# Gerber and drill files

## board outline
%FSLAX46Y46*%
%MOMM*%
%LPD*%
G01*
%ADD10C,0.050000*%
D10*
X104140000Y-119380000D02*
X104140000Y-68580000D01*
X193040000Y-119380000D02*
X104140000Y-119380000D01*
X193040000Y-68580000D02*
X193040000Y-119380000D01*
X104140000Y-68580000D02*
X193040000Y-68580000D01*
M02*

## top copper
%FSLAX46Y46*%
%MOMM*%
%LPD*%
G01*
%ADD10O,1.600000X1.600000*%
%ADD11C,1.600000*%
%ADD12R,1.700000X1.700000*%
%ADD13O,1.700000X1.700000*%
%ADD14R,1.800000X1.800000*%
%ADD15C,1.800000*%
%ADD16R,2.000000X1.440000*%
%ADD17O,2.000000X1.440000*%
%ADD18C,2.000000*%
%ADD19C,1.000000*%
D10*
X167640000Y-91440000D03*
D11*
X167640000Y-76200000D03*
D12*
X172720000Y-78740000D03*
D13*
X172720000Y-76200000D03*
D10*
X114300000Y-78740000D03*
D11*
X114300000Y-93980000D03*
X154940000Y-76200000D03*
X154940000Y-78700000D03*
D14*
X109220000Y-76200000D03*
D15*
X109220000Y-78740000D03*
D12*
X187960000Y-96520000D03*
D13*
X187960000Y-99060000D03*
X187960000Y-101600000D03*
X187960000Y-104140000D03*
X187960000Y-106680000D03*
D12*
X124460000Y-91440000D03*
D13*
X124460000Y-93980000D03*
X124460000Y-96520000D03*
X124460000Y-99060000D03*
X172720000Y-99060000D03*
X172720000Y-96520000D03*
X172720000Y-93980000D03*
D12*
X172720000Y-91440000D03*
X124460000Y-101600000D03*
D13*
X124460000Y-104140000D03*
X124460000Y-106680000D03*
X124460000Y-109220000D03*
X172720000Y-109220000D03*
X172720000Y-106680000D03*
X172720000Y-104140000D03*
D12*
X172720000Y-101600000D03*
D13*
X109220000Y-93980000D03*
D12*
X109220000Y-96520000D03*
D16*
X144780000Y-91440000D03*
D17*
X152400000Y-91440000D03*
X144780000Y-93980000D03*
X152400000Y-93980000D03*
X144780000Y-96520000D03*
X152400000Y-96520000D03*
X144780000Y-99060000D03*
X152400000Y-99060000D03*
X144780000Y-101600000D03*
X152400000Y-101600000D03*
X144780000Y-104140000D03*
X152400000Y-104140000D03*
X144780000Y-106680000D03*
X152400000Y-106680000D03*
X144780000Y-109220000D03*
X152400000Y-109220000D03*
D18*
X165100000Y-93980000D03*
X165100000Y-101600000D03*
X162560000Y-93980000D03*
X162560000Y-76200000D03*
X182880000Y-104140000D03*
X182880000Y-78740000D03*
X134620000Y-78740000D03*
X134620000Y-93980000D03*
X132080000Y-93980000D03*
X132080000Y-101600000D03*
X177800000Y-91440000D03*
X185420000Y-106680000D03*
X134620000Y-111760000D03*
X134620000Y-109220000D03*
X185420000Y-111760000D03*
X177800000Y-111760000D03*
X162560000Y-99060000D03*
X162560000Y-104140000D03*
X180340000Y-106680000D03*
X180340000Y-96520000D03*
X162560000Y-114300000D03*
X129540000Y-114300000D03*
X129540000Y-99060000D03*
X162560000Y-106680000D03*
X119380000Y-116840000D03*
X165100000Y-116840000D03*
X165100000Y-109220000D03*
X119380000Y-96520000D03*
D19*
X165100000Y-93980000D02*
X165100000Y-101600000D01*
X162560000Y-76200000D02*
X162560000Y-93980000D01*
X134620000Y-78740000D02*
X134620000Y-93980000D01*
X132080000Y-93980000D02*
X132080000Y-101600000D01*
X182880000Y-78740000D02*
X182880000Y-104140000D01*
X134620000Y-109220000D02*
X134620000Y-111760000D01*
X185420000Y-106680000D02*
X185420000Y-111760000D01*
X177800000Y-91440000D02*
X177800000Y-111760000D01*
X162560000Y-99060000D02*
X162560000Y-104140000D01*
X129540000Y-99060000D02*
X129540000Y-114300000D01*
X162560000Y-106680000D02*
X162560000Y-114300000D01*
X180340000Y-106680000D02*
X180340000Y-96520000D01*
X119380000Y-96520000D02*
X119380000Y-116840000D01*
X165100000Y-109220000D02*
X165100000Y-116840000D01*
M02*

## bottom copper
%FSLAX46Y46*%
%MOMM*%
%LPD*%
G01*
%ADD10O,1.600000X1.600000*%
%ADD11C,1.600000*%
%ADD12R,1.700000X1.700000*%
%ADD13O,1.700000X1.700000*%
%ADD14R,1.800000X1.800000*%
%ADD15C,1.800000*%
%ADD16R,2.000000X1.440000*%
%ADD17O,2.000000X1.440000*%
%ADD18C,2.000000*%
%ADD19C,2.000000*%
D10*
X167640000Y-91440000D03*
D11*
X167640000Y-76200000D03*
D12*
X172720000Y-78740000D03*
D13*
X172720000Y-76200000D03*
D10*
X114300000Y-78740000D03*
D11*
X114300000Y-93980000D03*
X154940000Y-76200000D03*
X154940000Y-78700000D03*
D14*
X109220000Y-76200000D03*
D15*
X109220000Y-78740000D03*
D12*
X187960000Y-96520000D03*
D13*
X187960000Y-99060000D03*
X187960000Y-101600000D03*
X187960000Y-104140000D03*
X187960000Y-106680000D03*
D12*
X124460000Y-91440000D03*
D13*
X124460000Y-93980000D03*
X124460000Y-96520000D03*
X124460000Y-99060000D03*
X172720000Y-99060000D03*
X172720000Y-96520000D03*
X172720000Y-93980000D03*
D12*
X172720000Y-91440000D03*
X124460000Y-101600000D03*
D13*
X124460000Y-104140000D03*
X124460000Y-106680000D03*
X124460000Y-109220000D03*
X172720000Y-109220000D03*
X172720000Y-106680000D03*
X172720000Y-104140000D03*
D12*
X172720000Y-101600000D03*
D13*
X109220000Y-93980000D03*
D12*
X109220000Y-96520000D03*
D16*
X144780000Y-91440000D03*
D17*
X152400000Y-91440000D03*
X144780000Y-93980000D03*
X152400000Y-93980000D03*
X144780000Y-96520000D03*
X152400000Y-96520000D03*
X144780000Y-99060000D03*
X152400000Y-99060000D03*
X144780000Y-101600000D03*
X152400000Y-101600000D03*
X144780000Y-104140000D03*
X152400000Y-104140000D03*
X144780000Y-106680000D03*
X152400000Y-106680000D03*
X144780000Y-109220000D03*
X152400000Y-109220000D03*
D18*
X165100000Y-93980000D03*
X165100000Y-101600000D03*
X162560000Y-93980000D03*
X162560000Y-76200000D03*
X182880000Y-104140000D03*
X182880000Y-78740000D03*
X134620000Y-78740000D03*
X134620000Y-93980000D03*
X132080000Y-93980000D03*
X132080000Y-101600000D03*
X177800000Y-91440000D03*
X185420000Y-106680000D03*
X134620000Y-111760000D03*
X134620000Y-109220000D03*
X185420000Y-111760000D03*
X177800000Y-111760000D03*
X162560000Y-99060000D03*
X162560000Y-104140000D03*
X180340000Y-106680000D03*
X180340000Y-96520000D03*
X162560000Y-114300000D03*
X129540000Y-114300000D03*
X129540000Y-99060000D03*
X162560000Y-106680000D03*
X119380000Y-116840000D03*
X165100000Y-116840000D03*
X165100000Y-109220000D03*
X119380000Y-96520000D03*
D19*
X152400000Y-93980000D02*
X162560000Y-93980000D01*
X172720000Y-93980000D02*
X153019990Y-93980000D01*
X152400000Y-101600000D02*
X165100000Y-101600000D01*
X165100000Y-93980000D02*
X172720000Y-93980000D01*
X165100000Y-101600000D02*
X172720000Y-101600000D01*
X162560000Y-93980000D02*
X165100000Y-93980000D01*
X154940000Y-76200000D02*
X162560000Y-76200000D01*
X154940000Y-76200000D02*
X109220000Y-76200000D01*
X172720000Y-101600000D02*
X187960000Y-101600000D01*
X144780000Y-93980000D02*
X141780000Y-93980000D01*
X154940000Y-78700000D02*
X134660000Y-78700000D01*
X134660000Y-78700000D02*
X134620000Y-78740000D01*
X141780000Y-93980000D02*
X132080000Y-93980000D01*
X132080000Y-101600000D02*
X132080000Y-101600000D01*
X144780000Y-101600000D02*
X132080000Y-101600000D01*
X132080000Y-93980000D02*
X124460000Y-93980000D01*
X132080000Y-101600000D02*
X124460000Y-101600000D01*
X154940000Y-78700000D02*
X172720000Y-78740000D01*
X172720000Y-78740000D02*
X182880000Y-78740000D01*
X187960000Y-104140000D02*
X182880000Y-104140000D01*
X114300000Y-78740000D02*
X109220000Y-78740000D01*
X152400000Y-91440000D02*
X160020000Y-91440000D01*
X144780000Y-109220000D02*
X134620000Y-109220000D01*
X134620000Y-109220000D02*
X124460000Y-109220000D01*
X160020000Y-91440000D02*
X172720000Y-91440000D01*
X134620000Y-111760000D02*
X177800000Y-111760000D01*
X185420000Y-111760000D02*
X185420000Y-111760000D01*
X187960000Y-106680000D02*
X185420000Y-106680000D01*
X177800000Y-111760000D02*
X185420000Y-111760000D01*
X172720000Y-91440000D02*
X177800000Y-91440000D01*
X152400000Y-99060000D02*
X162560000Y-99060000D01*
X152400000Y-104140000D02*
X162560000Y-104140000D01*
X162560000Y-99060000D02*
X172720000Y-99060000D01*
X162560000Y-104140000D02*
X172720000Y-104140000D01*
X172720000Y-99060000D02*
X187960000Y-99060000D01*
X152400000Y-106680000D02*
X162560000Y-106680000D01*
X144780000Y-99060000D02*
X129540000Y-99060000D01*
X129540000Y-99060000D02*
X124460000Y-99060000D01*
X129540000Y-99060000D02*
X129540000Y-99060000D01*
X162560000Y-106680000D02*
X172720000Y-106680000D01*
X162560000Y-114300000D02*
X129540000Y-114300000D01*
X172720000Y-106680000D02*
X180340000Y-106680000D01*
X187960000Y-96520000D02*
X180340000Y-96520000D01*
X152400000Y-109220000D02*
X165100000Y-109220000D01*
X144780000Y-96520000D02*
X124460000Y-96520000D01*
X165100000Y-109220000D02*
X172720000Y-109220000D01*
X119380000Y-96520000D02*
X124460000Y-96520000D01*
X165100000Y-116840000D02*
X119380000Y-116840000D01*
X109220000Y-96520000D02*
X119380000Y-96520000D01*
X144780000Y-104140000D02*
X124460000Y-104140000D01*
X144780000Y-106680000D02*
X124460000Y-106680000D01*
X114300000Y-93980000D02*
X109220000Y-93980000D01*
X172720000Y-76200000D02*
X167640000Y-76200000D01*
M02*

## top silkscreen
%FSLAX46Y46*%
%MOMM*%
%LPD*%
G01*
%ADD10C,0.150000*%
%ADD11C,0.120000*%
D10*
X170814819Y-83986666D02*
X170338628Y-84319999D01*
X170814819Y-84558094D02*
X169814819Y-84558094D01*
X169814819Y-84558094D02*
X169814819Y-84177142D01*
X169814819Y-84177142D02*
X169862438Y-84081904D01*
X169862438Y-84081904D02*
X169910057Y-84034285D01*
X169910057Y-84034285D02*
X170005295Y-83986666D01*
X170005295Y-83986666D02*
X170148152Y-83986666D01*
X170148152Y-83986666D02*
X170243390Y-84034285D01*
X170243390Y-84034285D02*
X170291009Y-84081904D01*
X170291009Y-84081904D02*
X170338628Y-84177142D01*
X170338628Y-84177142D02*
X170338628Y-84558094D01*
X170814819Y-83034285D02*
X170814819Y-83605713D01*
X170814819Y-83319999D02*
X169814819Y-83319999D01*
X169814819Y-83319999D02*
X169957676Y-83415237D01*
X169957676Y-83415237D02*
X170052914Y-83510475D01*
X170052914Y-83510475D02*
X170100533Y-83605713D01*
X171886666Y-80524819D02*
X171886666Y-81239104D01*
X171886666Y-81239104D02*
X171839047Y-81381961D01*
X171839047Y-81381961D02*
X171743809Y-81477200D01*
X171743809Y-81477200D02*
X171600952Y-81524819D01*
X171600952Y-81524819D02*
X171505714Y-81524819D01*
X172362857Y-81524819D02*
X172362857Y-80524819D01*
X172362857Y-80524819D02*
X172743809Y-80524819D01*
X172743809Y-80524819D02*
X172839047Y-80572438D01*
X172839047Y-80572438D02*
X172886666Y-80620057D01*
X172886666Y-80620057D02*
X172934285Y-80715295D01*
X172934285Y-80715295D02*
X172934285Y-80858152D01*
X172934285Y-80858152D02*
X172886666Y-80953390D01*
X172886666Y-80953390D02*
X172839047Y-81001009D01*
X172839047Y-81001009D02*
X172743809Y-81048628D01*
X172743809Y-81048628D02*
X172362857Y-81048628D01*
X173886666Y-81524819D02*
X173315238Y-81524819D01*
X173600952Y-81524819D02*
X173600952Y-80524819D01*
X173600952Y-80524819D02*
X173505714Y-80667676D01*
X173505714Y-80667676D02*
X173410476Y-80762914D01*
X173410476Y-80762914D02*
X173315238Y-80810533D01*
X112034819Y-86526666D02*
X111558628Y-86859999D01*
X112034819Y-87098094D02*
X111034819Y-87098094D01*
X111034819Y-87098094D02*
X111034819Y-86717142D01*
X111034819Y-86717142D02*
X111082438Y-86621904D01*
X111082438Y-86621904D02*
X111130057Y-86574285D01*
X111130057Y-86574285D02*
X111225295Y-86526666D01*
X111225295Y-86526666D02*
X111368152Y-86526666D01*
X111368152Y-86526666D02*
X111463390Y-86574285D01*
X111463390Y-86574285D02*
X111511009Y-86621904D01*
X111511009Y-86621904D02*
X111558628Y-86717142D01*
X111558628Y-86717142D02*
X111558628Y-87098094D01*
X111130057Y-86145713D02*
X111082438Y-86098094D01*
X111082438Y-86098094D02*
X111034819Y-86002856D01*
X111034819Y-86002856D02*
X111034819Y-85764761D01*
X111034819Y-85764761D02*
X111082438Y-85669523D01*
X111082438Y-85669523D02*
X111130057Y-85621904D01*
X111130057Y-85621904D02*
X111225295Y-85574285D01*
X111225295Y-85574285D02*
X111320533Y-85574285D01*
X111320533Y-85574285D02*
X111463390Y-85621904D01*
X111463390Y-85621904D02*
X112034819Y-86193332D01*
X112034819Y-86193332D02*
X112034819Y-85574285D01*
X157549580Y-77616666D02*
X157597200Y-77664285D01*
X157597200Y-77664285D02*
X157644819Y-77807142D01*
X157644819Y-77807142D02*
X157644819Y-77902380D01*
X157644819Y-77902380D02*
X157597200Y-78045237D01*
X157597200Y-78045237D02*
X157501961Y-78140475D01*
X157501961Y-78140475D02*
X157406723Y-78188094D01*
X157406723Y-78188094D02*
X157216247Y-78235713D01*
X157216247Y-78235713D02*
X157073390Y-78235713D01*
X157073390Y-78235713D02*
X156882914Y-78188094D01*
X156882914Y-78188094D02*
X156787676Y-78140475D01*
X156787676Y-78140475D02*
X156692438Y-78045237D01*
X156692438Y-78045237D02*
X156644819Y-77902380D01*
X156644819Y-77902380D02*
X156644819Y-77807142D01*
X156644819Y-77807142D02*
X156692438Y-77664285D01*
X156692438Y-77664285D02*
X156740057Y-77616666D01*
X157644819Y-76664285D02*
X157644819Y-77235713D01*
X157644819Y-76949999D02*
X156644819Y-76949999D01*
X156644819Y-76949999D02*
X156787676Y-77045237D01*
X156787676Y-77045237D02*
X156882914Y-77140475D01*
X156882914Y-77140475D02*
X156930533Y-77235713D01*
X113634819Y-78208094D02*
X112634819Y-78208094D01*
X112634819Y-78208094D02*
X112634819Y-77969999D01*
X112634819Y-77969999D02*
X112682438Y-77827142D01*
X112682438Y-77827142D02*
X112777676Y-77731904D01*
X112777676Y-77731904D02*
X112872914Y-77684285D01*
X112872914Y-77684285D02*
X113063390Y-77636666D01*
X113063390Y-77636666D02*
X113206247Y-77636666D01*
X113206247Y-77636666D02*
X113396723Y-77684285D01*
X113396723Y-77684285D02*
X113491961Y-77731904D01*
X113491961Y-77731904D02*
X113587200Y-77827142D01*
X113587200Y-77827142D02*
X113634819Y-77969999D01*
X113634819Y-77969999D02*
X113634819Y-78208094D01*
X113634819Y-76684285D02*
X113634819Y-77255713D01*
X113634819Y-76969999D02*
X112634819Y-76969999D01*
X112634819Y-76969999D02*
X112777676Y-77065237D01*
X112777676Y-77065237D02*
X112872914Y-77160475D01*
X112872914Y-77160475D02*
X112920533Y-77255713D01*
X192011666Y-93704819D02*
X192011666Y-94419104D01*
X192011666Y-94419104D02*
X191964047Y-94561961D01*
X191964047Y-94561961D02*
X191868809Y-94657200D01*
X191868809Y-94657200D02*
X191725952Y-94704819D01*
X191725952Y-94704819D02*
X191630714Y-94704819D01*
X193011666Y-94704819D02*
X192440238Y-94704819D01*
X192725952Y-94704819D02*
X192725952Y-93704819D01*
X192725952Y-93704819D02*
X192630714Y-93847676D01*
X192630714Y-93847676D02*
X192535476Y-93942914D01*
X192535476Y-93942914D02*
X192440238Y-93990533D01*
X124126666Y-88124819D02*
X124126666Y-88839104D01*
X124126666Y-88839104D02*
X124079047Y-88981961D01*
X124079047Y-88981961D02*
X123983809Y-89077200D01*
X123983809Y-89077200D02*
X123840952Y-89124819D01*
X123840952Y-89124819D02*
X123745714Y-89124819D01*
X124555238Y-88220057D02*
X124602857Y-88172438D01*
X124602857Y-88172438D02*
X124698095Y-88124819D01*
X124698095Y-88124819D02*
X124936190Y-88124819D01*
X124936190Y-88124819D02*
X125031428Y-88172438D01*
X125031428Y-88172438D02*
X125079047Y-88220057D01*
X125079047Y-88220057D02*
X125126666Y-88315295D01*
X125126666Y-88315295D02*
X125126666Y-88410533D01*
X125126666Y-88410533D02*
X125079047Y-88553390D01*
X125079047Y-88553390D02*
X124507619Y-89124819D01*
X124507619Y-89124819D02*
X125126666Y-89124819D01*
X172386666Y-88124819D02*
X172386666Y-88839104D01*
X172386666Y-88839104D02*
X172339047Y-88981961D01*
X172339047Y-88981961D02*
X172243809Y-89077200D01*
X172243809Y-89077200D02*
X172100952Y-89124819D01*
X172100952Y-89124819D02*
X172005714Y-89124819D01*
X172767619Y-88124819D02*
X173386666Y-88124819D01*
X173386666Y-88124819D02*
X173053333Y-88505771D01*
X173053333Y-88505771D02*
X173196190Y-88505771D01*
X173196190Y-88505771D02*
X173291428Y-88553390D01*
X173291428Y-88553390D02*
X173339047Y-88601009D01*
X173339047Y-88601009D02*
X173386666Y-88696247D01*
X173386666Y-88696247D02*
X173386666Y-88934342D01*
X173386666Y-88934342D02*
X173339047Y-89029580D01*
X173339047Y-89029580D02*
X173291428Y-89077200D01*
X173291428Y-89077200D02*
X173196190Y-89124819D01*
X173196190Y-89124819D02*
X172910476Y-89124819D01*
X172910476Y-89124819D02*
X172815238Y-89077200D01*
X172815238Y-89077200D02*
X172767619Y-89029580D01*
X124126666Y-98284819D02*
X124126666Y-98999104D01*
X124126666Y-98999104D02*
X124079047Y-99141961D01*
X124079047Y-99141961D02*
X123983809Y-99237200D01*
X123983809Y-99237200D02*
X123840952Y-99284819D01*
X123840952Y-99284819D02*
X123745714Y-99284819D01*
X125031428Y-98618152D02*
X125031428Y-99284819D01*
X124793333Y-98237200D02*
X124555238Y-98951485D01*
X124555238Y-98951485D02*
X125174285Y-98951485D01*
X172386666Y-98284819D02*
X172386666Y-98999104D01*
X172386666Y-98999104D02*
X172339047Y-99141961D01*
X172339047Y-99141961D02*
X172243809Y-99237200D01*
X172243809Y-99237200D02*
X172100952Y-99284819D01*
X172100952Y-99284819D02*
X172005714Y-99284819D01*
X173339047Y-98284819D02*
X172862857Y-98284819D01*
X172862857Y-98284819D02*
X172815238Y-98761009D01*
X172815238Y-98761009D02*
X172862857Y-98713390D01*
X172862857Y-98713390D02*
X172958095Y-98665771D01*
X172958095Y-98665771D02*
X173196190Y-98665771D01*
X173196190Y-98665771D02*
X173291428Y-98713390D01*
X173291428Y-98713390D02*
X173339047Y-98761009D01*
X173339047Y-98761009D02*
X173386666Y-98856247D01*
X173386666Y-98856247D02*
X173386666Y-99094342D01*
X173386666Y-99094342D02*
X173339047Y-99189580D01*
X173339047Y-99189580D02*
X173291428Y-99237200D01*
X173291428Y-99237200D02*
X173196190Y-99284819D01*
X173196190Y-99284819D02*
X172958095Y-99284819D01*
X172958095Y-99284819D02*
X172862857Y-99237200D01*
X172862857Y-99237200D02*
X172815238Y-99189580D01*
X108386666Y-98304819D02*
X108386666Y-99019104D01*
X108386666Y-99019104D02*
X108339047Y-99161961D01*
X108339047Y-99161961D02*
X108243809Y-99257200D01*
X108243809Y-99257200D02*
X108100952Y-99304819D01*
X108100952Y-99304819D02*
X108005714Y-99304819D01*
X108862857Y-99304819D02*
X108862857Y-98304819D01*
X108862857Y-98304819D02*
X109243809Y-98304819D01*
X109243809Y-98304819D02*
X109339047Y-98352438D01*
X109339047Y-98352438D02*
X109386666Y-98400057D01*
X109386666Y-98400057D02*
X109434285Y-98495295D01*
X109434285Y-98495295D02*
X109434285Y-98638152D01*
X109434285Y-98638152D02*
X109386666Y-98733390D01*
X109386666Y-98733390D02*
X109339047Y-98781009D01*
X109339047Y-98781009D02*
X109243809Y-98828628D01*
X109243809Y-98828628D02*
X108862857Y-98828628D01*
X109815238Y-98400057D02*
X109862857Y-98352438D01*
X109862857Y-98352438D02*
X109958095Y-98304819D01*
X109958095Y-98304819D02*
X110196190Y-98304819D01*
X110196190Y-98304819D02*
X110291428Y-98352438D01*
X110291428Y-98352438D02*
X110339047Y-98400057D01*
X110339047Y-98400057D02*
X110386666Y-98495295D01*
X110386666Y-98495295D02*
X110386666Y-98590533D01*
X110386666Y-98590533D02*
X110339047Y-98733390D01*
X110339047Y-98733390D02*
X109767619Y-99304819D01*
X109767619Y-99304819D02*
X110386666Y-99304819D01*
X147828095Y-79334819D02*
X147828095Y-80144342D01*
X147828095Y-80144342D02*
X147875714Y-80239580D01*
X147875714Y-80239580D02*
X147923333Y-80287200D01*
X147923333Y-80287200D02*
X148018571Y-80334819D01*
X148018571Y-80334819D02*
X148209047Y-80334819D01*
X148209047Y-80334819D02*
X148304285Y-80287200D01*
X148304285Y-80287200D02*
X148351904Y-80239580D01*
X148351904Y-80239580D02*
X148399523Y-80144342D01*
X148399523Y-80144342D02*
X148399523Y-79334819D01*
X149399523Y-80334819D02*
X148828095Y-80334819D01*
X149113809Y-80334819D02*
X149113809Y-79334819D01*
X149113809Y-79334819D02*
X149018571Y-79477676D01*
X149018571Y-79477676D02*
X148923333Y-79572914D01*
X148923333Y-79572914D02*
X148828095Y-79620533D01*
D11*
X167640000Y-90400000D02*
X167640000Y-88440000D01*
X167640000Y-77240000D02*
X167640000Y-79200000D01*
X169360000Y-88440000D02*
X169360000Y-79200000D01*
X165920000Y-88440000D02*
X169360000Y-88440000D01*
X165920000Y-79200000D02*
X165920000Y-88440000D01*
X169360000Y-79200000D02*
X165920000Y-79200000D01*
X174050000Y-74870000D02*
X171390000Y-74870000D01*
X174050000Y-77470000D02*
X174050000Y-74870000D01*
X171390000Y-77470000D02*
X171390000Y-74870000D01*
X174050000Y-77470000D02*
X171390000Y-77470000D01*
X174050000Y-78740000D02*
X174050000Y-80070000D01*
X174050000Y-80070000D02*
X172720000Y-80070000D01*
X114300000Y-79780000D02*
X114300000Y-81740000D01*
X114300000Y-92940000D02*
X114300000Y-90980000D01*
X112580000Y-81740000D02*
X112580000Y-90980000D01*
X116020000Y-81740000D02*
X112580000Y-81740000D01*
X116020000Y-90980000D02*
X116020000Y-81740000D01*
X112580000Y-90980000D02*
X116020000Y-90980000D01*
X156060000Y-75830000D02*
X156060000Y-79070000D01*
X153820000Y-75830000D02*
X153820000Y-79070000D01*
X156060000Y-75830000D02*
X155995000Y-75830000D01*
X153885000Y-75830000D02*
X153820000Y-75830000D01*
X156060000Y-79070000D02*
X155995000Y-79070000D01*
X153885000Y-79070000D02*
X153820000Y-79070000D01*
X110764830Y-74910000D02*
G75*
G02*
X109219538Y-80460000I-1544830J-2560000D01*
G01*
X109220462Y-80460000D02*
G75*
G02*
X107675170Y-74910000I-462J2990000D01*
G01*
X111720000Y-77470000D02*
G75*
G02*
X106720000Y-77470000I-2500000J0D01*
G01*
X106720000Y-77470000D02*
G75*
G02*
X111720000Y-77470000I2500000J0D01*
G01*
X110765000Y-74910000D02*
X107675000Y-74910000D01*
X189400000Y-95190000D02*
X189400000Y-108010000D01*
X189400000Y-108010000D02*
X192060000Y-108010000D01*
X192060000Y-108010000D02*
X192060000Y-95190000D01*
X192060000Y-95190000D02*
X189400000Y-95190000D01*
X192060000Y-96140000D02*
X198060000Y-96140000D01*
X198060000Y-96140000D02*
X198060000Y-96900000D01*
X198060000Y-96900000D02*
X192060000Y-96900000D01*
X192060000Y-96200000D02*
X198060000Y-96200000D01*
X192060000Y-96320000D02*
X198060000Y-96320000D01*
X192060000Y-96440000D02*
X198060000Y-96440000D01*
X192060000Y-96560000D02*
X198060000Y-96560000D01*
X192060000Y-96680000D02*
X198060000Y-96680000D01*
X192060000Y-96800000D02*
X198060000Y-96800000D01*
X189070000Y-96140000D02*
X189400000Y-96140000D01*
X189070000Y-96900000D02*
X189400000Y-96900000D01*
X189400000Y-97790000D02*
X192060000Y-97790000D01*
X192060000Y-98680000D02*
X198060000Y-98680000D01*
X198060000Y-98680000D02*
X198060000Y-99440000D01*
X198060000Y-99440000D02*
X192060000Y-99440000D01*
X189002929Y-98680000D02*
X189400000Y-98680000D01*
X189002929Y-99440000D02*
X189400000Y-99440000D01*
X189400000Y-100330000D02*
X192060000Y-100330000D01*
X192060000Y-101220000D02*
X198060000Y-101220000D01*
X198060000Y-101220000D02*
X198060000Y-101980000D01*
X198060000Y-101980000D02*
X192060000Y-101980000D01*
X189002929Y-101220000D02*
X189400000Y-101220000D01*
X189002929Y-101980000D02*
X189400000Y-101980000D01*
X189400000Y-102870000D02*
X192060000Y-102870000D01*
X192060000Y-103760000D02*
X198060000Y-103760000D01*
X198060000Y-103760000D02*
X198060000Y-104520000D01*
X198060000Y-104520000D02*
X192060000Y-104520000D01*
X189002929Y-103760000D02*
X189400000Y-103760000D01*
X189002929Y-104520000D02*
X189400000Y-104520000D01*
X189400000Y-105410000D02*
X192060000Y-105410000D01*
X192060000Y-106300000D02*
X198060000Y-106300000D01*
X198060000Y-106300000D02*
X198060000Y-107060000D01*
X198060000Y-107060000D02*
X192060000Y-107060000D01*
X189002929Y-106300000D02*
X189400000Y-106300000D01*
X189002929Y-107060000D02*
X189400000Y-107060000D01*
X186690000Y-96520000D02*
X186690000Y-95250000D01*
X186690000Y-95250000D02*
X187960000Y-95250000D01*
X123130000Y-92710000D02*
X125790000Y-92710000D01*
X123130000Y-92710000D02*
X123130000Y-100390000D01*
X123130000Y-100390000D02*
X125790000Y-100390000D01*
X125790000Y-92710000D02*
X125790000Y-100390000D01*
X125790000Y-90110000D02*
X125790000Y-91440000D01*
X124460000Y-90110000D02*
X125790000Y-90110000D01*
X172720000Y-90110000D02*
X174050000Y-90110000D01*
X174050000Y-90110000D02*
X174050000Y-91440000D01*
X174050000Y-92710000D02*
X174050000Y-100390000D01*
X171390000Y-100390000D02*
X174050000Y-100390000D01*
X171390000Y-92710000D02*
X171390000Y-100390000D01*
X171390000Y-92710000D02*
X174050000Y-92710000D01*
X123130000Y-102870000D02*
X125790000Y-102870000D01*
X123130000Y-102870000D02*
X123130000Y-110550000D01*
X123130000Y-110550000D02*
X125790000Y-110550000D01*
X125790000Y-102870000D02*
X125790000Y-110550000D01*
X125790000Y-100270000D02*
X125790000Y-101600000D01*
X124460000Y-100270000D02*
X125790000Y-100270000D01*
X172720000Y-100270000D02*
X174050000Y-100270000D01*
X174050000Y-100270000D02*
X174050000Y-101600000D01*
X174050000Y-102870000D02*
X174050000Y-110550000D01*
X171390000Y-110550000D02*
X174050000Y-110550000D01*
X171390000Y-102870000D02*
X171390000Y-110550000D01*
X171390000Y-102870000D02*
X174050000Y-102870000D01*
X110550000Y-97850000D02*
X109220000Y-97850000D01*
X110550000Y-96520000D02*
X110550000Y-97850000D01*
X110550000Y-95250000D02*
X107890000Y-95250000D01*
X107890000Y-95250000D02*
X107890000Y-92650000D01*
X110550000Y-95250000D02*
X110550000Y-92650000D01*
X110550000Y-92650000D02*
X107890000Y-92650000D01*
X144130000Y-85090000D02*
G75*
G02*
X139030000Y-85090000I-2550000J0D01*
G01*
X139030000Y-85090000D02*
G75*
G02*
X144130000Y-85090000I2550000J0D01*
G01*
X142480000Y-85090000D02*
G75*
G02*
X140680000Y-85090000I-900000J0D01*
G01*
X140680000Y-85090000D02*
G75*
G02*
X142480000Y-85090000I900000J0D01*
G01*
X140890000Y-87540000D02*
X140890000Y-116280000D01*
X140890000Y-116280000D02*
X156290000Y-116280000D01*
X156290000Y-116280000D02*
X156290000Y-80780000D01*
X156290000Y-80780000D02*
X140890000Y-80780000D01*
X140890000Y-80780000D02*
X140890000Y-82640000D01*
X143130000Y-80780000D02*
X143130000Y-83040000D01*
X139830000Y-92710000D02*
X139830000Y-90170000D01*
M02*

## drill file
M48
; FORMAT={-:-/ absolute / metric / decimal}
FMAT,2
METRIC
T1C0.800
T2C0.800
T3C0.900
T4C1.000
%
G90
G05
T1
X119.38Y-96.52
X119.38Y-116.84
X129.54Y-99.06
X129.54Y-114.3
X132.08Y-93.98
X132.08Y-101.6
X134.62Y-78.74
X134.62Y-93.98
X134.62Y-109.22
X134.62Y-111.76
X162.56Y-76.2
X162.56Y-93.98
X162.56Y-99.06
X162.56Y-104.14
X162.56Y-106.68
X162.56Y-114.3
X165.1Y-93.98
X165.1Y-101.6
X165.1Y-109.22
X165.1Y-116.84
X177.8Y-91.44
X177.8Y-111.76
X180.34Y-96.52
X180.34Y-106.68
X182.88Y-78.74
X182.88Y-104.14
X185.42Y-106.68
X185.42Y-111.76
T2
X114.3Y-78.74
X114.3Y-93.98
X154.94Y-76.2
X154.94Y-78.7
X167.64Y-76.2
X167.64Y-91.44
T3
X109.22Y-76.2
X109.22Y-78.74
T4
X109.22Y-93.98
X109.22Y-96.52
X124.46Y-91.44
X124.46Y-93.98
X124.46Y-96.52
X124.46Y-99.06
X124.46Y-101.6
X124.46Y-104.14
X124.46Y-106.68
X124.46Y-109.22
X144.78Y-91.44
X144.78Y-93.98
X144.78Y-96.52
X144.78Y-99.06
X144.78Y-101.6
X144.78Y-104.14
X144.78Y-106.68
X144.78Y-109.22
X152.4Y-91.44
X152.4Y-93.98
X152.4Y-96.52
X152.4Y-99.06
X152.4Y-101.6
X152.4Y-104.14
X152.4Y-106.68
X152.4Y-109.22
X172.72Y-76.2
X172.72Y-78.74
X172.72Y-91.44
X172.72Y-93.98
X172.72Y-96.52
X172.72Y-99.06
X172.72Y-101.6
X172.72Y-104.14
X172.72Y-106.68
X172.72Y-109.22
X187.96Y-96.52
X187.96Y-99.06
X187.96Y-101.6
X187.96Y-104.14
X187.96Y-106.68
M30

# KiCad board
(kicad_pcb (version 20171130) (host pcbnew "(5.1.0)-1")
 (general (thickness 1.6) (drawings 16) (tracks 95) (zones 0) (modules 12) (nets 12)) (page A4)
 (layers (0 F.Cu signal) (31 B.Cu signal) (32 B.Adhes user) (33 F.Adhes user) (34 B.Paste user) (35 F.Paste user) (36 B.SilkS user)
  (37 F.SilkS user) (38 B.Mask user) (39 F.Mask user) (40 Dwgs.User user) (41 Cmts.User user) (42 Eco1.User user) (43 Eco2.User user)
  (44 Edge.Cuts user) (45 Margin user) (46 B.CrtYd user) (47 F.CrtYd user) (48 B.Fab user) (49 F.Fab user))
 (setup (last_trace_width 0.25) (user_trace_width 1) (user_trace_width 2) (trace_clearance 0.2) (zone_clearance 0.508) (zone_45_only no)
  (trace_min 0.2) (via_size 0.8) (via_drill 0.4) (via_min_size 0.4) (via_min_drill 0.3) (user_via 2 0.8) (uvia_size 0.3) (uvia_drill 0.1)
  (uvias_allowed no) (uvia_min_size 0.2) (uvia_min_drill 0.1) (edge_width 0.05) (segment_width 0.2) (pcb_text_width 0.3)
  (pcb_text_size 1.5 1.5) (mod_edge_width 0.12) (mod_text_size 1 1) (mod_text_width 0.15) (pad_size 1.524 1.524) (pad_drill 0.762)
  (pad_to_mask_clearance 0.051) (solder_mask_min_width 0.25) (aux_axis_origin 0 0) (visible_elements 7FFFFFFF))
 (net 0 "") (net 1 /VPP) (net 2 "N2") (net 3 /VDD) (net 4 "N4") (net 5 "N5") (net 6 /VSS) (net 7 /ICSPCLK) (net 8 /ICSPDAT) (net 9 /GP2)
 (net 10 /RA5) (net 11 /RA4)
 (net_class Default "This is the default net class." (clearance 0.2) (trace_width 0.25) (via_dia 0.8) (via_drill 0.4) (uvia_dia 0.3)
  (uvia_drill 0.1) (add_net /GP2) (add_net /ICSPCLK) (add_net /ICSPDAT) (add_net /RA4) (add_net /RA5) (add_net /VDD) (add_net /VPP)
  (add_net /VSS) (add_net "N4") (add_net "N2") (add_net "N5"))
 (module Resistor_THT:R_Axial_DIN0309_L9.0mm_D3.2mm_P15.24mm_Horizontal (layer F.Cu) (at 167.64 76.2 270)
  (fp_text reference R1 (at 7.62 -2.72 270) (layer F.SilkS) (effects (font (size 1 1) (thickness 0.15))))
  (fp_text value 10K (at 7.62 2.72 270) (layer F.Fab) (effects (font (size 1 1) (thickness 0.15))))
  (fp_line (start 14.2 0) (end 12.24 0) (layer F.SilkS) (width 0.12))
  (fp_line (start 1.04 0) (end 3 0) (layer F.SilkS) (width 0.12))
  (fp_line (start 12.24 -1.72) (end 3 -1.72) (layer F.SilkS) (width 0.12))
  (fp_line (start 12.24 1.72) (end 12.24 -1.72) (layer F.SilkS) (width 0.12))
  (fp_line (start 3 1.72) (end 12.24 1.72) (layer F.SilkS) (width 0.12))
  (fp_line (start 3 -1.72) (end 3 1.72) (layer F.SilkS) (width 0.12))
  (pad 2 thru_hole oval (at 15.24 0 270) (size 1.6 1.6) (drill 0.8) (layers *.Cu *.Mask) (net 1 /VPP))
  (pad 1 thru_hole circle (at 0 0 270) (size 1.6 1.6) (drill 0.8) (layers *.Cu *.Mask) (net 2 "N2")))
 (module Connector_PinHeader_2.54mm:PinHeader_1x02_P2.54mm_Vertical (layer F.Cu) (at 172.72 78.74 180)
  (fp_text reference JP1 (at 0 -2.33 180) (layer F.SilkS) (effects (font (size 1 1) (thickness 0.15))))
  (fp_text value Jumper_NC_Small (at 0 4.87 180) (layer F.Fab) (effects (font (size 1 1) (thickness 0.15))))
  (fp_line (start -1.33 3.87) (end 1.33 3.87) (layer F.SilkS) (width 0.12))
  (fp_line (start -1.33 1.27) (end -1.33 3.87) (layer F.SilkS) (width 0.12))
  (fp_line (start 1.33 1.27) (end 1.33 3.87) (layer F.SilkS) (width 0.12))
  (fp_line (start -1.33 1.27) (end 1.33 1.27) (layer F.SilkS) (width 0.12))
  (fp_line (start -1.33 0) (end -1.33 -1.33) (layer F.SilkS) (width 0.12))
  (fp_line (start -1.33 -1.33) (end 0 -1.33) (layer F.SilkS) (width 0.12))
  (pad 1 thru_hole rect (at 0 0 180) (size 1.7 1.7) (drill 1) (layers *.Cu *.Mask) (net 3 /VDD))
  (pad 2 thru_hole oval (at 0 2.54 180) (size 1.7 1.7) (drill 1) (layers *.Cu *.Mask) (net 2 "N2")))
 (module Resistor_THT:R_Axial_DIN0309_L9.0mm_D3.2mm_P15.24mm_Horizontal (layer F.Cu) (at 114.3 93.98 90)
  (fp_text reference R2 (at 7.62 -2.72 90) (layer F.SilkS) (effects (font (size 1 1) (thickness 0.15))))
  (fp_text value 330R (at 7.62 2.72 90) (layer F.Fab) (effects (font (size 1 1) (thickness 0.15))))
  (fp_line (start 14.2 0) (end 12.24 0) (layer F.SilkS) (width 0.12))
  (fp_line (start 1.04 0) (end 3 0) (layer F.SilkS) (width 0.12))
  (fp_line (start 12.24 -1.72) (end 3 -1.72) (layer F.SilkS) (width 0.12))
  (fp_line (start 12.24 1.72) (end 12.24 -1.72) (layer F.SilkS) (width 0.12))
  (fp_line (start 3 1.72) (end 12.24 1.72) (layer F.SilkS) (width 0.12))
  (fp_line (start 3 -1.72) (end 3 1.72) (layer F.SilkS) (width 0.12))
  (pad 2 thru_hole oval (at 15.24 0 90) (size 1.6 1.6) (drill 0.8) (layers *.Cu *.Mask) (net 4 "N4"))
  (pad 1 thru_hole circle (at 0 0 90) (size 1.6 1.6) (drill 0.8) (layers *.Cu *.Mask) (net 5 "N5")))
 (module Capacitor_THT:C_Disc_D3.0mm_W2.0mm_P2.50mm (layer F.Cu) (at 154.94 76.2 270)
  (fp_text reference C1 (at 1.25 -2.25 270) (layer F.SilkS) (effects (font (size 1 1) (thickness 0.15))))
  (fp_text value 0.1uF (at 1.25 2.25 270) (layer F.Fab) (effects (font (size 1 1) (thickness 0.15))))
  (fp_line (start -0.37 -1.12) (end 2.87 -1.12) (layer F.SilkS) (width 0.12))
  (fp_line (start -0.37 1.12) (end 2.87 1.12) (layer F.SilkS) (width 0.12))
  (fp_line (start -0.37 -1.12) (end -0.37 -1.055) (layer F.SilkS) (width 0.12))
  (fp_line (start -0.37 1.055) (end -0.37 1.12) (layer F.SilkS) (width 0.12))
  (fp_line (start 2.87 -1.12) (end 2.87 -1.055) (layer F.SilkS) (width 0.12))
  (fp_line (start 2.87 1.055) (end 2.87 1.12) (layer F.SilkS) (width 0.12))
  (pad 1 thru_hole circle (at 0 0 270) (size 1.6 1.6) (drill 0.8) (layers *.Cu *.Mask) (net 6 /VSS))
  (pad 2 thru_hole circle (at 2.5 0 270) (size 1.6 1.6) (drill 0.8) (layers *.Cu *.Mask) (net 3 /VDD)))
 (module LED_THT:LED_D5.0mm (layer F.Cu) (at 109.22 76.2 270)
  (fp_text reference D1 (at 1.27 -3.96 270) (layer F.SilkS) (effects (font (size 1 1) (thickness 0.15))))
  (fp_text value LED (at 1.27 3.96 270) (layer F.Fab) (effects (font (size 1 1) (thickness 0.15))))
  (fp_arc (start 1.27 0) (end -1.29 -1.54483) (angle 148.9) (layer F.SilkS) (width 0.12))
  (fp_arc (start 1.27 0) (end -1.29 1.54483) (angle -148.9) (layer F.SilkS) (width 0.12))
  (fp_circle (center 1.27 0) (end 3.77 0) (layer F.SilkS) (width 0.12))
  (fp_line (start -1.29 -1.545) (end -1.29 1.545) (layer F.SilkS) (width 0.12))
  (pad 1 thru_hole rect (at 0 0 270) (size 1.8 1.8) (drill 0.9) (layers *.Cu *.Mask) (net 6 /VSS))
  (pad 2 thru_hole circle (at 2.54 0 270) (size 1.8 1.8) (drill 0.9) (layers *.Cu *.Mask) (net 4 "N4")))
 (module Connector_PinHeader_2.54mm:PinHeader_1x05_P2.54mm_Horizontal (layer F.Cu) (at 187.96 96.52)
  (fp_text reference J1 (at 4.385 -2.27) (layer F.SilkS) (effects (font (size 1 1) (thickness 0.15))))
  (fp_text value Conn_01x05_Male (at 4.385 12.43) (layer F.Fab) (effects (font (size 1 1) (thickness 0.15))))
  (fp_line (start 1.44 -1.33) (end 1.44 11.49) (layer F.SilkS) (width 0.12))
  (fp_line (start 1.44 11.49) (end 4.1 11.49) (layer F.SilkS) (width 0.12))
  (fp_line (start 4.1 11.49) (end 4.1 -1.33) (layer F.SilkS) (width 0.12))
  (fp_line (start 4.1 -1.33) (end 1.44 -1.33) (layer F.SilkS) (width 0.12))
  (fp_line (start 4.1 -0.38) (end 10.1 -0.38) (layer F.SilkS) (width 0.12))
  (fp_line (start 10.1 -0.38) (end 10.1 0.38) (layer F.SilkS) (width 0.12))
  (fp_line (start 10.1 0.38) (end 4.1 0.38) (layer F.SilkS) (width 0.12))
  (fp_line (start 4.1 -0.32) (end 10.1 -0.32) (layer F.SilkS) (width 0.12))
  (fp_line (start 4.1 -0.2) (end 10.1 -0.2) (layer F.SilkS) (width 0.12))
  (fp_line (start 4.1 -0.08) (end 10.1 -0.08) (layer F.SilkS) (width 0.12))
  (fp_line (start 4.1 0.04) (end 10.1 0.04) (layer F.SilkS) (width 0.12))
  (fp_line (start 4.1 0.16) (end 10.1 0.16) (layer F.SilkS) (width 0.12))
  (fp_line (start 4.1 0.28) (end 10.1 0.28) (layer F.SilkS) (width 0.12))
  (fp_line (start 1.11 -0.38) (end 1.44 -0.38) (layer F.SilkS) (width 0.12))
  (fp_line (start 1.11 0.38) (end 1.44 0.38) (layer F.SilkS) (width 0.12))
  (fp_line (start 1.44 1.27) (end 4.1 1.27) (layer F.SilkS) (width 0.12))
  (fp_line (start 4.1 2.16) (end 10.1 2.16) (layer F.SilkS) (width 0.12))
  (fp_line (start 10.1 2.16) (end 10.1 2.92) (layer F.SilkS) (width 0.12))
  (fp_line (start 10.1 2.92) (end 4.1 2.92) (layer F.SilkS) (width 0.12))
  (fp_line (start 1.042929 2.16) (end 1.44 2.16) (layer F.SilkS) (width 0.12))
  (fp_line (start 1.042929 2.92) (end 1.44 2.92) (layer F.SilkS) (width 0.12))
  (fp_line (start 1.44 3.81) (end 4.1 3.81) (layer F.SilkS) (width 0.12))
  (fp_line (start 4.1 4.7) (end 10.1 4.7) (layer F.SilkS) (width 0.12))
  (fp_line (start 10.1 4.7) (end 10.1 5.46) (layer F.SilkS) (width 0.12))
  (fp_line (start 10.1 5.46) (end 4.1 5.46) (layer F.SilkS) (width 0.12))
  (fp_line (start 1.042929 4.7) (end 1.44 4.7) (layer F.SilkS) (width 0.12))
  (fp_line (start 1.042929 5.46) (end 1.44 5.46) (layer F.SilkS) (width 0.12))
  (fp_line (start 1.44 6.35) (end 4.1 6.35) (layer F.SilkS) (width 0.12))
  (fp_line (start 4.1 7.24) (end 10.1 7.24) (layer F.SilkS) (width 0.12))
  (fp_line (start 10.1 7.24) (end 10.1 8) (layer F.SilkS) (width 0.12))
  (fp_line (start 10.1 8) (end 4.1 8) (layer F.SilkS) (width 0.12))
  (fp_line (start 1.042929 7.24) (end 1.44 7.24) (layer F.SilkS) (width 0.12))
  (fp_line (start 1.042929 8) (end 1.44 8) (layer F.SilkS) (width 0.12))
  (fp_line (start 1.44 8.89) (end 4.1 8.89) (layer F.SilkS) (width 0.12))
  (fp_line (start 4.1 9.78) (end 10.1 9.78) (layer F.SilkS) (width 0.12))
  (fp_line (start 10.1 9.78) (end 10.1 10.54) (layer F.SilkS) (width 0.12))
  (fp_line (start 10.1 10.54) (end 4.1 10.54) (layer F.SilkS) (width 0.12))
  (fp_line (start 1.042929 9.78) (end 1.44 9.78) (layer F.SilkS) (width 0.12))
  (fp_line (start 1.042929 10.54) (end 1.44 10.54) (layer F.SilkS) (width 0.12))
  (fp_line (start -1.27 0) (end -1.27 -1.27) (layer F.SilkS) (width 0.12))
  (fp_line (start -1.27 -1.27) (end 0 -1.27) (layer F.SilkS) (width 0.12))
  (pad 1 thru_hole rect (at 0 0) (size 1.7 1.7) (drill 1) (layers *.Cu *.Mask) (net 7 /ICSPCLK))
  (pad 2 thru_hole oval (at 0 2.54) (size 1.7 1.7) (drill 1) (layers *.Cu *.Mask) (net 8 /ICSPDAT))
  (pad 3 thru_hole oval (at 0 5.08) (size 1.7 1.7) (drill 1) (layers *.Cu *.Mask) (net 6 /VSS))
  (pad 4 thru_hole oval (at 0 7.62) (size 1.7 1.7) (drill 1) (layers *.Cu *.Mask) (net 3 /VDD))
  (pad 5 thru_hole oval (at 0 10.16) (size 1.7 1.7) (drill 1) (layers *.Cu *.Mask) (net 1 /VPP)))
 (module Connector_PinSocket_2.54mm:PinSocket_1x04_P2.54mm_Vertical (layer F.Cu) (at 124.46 91.44)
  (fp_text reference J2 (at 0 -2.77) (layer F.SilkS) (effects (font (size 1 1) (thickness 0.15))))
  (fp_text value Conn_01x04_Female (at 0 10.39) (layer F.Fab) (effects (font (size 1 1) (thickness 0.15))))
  (fp_line (start -1.33 1.27) (end 1.33 1.27) (layer F.SilkS) (width 0.12))
  (fp_line (start -1.33 1.27) (end -1.33 8.95) (layer F.SilkS) (width 0.12))
  (fp_line (start -1.33 8.95) (end 1.33 8.95) (layer F.SilkS) (width 0.12))
  (fp_line (start 1.33 1.27) (end 1.33 8.95) (layer F.SilkS) (width 0.12))
  (fp_line (start 1.33 -1.33) (end 1.33 0) (layer F.SilkS) (width 0.12))
  (fp_line (start 0 -1.33) (end 1.33 -1.33) (layer F.SilkS) (width 0.12))
  (pad 1 thru_hole rect (at 0 0) (size 1.7 1.7) (drill 1) (layers *.Cu *.Mask))
  (pad 2 thru_hole oval (at 0 2.54) (size 1.7 1.7) (drill 1) (layers *.Cu *.Mask) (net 3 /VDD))
  (pad 3 thru_hole oval (at 0 5.08) (size 1.7 1.7) (drill 1) (layers *.Cu *.Mask) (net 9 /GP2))
  (pad 4 thru_hole oval (at 0 7.62) (size 1.7 1.7) (drill 1) (layers *.Cu *.Mask) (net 7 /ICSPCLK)))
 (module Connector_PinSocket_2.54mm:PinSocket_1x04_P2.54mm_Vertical (layer F.Cu) (at 172.72 91.44)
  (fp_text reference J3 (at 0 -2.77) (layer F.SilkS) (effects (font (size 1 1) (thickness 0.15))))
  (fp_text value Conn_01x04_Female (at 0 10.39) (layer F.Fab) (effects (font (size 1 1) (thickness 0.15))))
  (fp_line (start 0 -1.33) (end 1.33 -1.33) (layer F.SilkS) (width 0.12))
  (fp_line (start 1.33 -1.33) (end 1.33 0) (layer F.SilkS) (width 0.12))
  (fp_line (start 1.33 1.27) (end 1.33 8.95) (layer F.SilkS) (width 0.12))
  (fp_line (start -1.33 8.95) (end 1.33 8.95) (layer F.SilkS) (width 0.12))
  (fp_line (start -1.33 1.27) (end -1.33 8.95) (layer F.SilkS) (width 0.12))
  (fp_line (start -1.33 1.27) (end 1.33 1.27) (layer F.SilkS) (width 0.12))
  (pad 4 thru_hole oval (at 0 7.62) (size 1.7 1.7) (drill 1) (layers *.Cu *.Mask) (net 8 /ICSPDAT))
  (pad 3 thru_hole oval (at 0 5.08) (size 1.7 1.7) (drill 1) (layers *.Cu *.Mask))
  (pad 2 thru_hole oval (at 0 2.54) (size 1.7 1.7) (drill 1) (layers *.Cu *.Mask) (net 6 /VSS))
  (pad 1 thru_hole rect (at 0 0) (size 1.7 1.7) (drill 1) (layers *.Cu *.Mask) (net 1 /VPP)))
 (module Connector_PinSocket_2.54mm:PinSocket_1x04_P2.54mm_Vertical (layer F.Cu) (at 124.46 101.6)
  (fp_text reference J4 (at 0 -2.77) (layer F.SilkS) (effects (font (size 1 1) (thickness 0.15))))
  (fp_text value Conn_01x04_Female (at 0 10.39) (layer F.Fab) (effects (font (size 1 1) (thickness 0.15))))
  (fp_line (start -1.33 1.27) (end 1.33 1.27) (layer F.SilkS) (width 0.12))
  (fp_line (start -1.33 1.27) (end -1.33 8.95) (layer F.SilkS) (width 0.12))
  (fp_line (start -1.33 8.95) (end 1.33 8.95) (layer F.SilkS) (width 0.12))
  (fp_line (start 1.33 1.27) (end 1.33 8.95) (layer F.SilkS) (width 0.12))
  (fp_line (start 1.33 -1.33) (end 1.33 0) (layer F.SilkS) (width 0.12))
  (fp_line (start 0 -1.33) (end 1.33 -1.33) (layer F.SilkS) (width 0.12))
  (pad 1 thru_hole rect (at 0 0) (size 1.7 1.7) (drill 1) (layers *.Cu *.Mask) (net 3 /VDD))
  (pad 2 thru_hole oval (at 0 2.54) (size 1.7 1.7) (drill 1) (layers *.Cu *.Mask) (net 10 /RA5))
  (pad 3 thru_hole oval (at 0 5.08) (size 1.7 1.7) (drill 1) (layers *.Cu *.Mask) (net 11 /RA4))
  (pad 4 thru_hole oval (at 0 7.62) (size 1.7 1.7) (drill 1) (layers *.Cu *.Mask) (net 1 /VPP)))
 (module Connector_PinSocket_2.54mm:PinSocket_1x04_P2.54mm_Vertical (layer F.Cu) (at 172.72 101.6)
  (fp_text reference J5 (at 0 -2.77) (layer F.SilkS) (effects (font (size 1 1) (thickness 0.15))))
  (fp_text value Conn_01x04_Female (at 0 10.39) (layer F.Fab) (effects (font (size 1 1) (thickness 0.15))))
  (fp_line (start 0 -1.33) (end 1.33 -1.33) (layer F.SilkS) (width 0.12))
  (fp_line (start 1.33 -1.33) (end 1.33 0) (layer F.SilkS) (width 0.12))
  (fp_line (start 1.33 1.27) (end 1.33 8.95) (layer F.SilkS) (width 0.12))
  (fp_line (start -1.33 8.95) (end 1.33 8.95) (layer F.SilkS) (width 0.12))
  (fp_line (start -1.33 1.27) (end -1.33 8.95) (layer F.SilkS) (width 0.12))
  (fp_line (start -1.33 1.27) (end 1.33 1.27) (layer F.SilkS) (width 0.12))
  (pad 4 thru_hole oval (at 0 7.62) (size 1.7 1.7) (drill 1) (layers *.Cu *.Mask) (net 9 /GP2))
  (pad 3 thru_hole oval (at 0 5.08) (size 1.7 1.7) (drill 1) (layers *.Cu *.Mask) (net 7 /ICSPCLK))
  (pad 2 thru_hole oval (at 0 2.54) (size 1.7 1.7) (drill 1) (layers *.Cu *.Mask) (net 8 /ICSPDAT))
  (pad 1 thru_hole rect (at 0 0) (size 1.7 1.7) (drill 1) (layers *.Cu *.Mask) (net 6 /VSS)))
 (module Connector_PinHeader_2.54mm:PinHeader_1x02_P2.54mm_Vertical (layer F.Cu) (at 109.22 96.52 180)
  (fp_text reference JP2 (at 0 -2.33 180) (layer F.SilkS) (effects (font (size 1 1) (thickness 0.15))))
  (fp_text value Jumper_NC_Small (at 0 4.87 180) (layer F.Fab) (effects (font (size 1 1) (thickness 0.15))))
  (fp_line (start -1.33 -1.33) (end 0 -1.33) (layer F.SilkS) (width 0.12))
  (fp_line (start -1.33 0) (end -1.33 -1.33) (layer F.SilkS) (width 0.12))
  (fp_line (start -1.33 1.27) (end 1.33 1.27) (layer F.SilkS) (width 0.12))
  (fp_line (start 1.33 1.27) (end 1.33 3.87) (layer F.SilkS) (width 0.12))
  (fp_line (start -1.33 1.27) (end -1.33 3.87) (layer F.SilkS) (width 0.12))
  (fp_line (start -1.33 3.87) (end 1.33 3.87) (layer F.SilkS) (width 0.12))
  (pad 2 thru_hole oval (at 0 2.54 180) (size 1.7 1.7) (drill 1) (layers *.Cu *.Mask) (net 5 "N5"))
  (pad 1 thru_hole rect (at 0 0 180) (size 1.7 1.7) (drill 1) (layers *.Cu *.Mask) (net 9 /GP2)))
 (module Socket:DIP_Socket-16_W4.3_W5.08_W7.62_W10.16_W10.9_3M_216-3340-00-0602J (layer F.Cu) (at 144.78 91.44)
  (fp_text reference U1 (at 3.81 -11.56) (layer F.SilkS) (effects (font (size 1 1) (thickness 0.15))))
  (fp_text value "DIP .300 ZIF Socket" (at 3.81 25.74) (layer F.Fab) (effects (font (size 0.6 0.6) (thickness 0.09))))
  (fp_circle (center -3.2 -6.35) (end -0.65 -6.35) (layer F.SilkS) (width 0.12))
  (fp_circle (center -3.2 -6.35) (end -2.3 -6.35) (layer F.SilkS) (width 0.12))
  (fp_line (start -3.89 -3.9) (end -3.89 24.84) (layer F.SilkS) (width 0.12))
  (fp_line (start -3.89 24.84) (end 11.51 24.84) (layer F.SilkS) (width 0.12))
  (fp_line (start 11.51 24.84) (end 11.51 -10.66) (layer F.SilkS) (width 0.12))
  (fp_line (start 11.51 -10.66) (end -3.89 -10.66) (layer F.SilkS) (width 0.12))
  (fp_line (start -3.89 -10.66) (end -3.89 -8.8) (layer F.SilkS) (width 0.12))
  (fp_line (start -1.65 -10.66) (end -1.65 -8.4) (layer F.SilkS) (width 0.12))
  (fp_line (start -4.95 1.27) (end -4.95 -1.27) (layer F.SilkS) (width 0.12))
  (pad 1 thru_hole rect (at 0 0) (size 2 1.44) (drill 1) (layers *.Cu *.Mask))
  (pad 16 thru_hole oval (at 7.62 0) (size 2 1.44) (drill 1) (layers *.Cu *.Mask) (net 1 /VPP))
  (pad 2 thru_hole oval (at 0 2.54) (size 2 1.44) (drill 1) (layers *.Cu *.Mask) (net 3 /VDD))
  (pad 15 thru_hole oval (at 7.62 2.54) (size 2 1.44) (drill 1) (layers *.Cu *.Mask) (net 6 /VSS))
  (pad 3 thru_hole oval (at 0 5.08) (size 2 1.44) (drill 1) (layers *.Cu *.Mask) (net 9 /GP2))
  (pad 14 thru_hole oval (at 7.62 5.08) (size 2 1.44) (drill 1) (layers *.Cu *.Mask))
  (pad 4 thru_hole oval (at 0 7.62) (size 2 1.44) (drill 1) (layers *.Cu *.Mask) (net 7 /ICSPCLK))
  (pad 13 thru_hole oval (at 7.62 7.62) (size 2 1.44) (drill 1) (layers *.Cu *.Mask) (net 8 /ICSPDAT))
  (pad 5 thru_hole oval (at 0 10.16) (size 2 1.44) (drill 1) (layers *.Cu *.Mask) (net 3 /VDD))
  (pad 12 thru_hole oval (at 7.62 10.16) (size 2 1.44) (drill 1) (layers *.Cu *.Mask) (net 6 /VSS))
  (pad 6 thru_hole oval (at 0 12.7) (size 2 1.44) (drill 1) (layers *.Cu *.Mask) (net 10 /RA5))
  (pad 11 thru_hole oval (at 7.62 12.7) (size 2 1.44) (drill 1) (layers *.Cu *.Mask) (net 8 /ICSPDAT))
  (pad 7 thru_hole oval (at 0 15.24) (size 2 1.44) (drill 1) (layers *.Cu *.Mask) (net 11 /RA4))
  (pad 10 thru_hole oval (at 7.62 15.24) (size 2 1.44) (drill 1) (layers *.Cu *.Mask) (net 7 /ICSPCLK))
  (pad 8 thru_hole oval (at 0 17.78) (size 2 1.44) (drill 1) (layers *.Cu *.Mask) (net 1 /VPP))
  (pad 9 thru_hole oval (at 7.62 17.78) (size 2 1.44) (drill 1) (layers *.Cu *.Mask) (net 9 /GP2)))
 (gr_line (start 104.14 119.38) (end 104.14 68.58) (layer Edge.Cuts) (width 0.05))
 (gr_line (start 193.04 119.38) (end 104.14 119.38) (layer Edge.Cuts) (width 0.05))
 (gr_line (start 193.04 68.58) (end 193.04 119.38) (layer Edge.Cuts) (width 0.05))
 (gr_line (start 104.14 68.58) (end 193.04 68.58) (layer Edge.Cuts) (width 0.05))
 (segment (start 152.4 93.98) (end 162.56 93.98) (width 2) (layer B.Cu) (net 6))
 (segment (start 172.72 93.98) (end 153.01999 93.98) (width 2) (layer B.Cu) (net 6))
 (segment (start 152.4 101.6) (end 165.1 101.6) (width 2) (layer B.Cu) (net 6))
 (segment (start 165.1 93.98) (end 172.72 93.98) (width 2) (layer B.Cu) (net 6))
 (via (at 165.1 93.98) (size 2) (drill 0.8) (layers F.Cu B.Cu) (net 6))
 (segment (start 165.1 101.6) (end 172.72 101.6) (width 2) (layer B.Cu) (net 6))
 (via (at 165.1 101.6) (size 2) (drill 0.8) (layers F.Cu B.Cu) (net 6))
 (segment (start 165.1 93.98) (end 165.1 101.6) (width 1) (layer F.Cu) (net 6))
 (segment (start 162.56 93.98) (end 165.1 93.98) (width 2) (layer B.Cu) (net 6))
 (via (at 162.56 93.98) (size 2) (drill 0.8) (layers F.Cu B.Cu) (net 6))
 (segment (start 154.94 76.2) (end 162.56 76.2) (width 2) (layer B.Cu) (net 6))
 (via (at 162.56 76.2) (size 2) (drill 0.8) (layers F.Cu B.Cu) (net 6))
 (segment (start 162.56 76.2) (end 162.56 93.98) (width 1) (layer F.Cu) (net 6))
 (segment (start 154.94 76.2) (end 109.22 76.2) (width 2) (layer B.Cu) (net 6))
 (segment (start 172.72 101.6) (end 187.96 101.6) (width 2) (layer B.Cu) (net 6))
 (via (at 182.88 104.14) (size 2) (drill 0.8) (layers F.Cu B.Cu) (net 3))
 (via (at 182.88 78.74) (size 2) (drill 0.8) (layers F.Cu B.Cu) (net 3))
 (segment (start 144.78 93.98) (end 141.78 93.98) (width 2) (layer B.Cu) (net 3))
 (via (at 134.62 78.74) (size 2) (drill 0.8) (layers F.Cu B.Cu) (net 3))
 (segment (start 154.94 78.7) (end 134.66 78.7) (width 2) (layer B.Cu) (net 3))
 (segment (start 134.66 78.7) (end 134.62 78.74) (width 2) (layer B.Cu) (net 3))
 (segment (start 134.62 78.74) (end 134.62 93.98) (width 1) (layer F.Cu) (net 3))
 (segment (start 141.78 93.98) (end 132.08 93.98) (width 2) (layer B.Cu) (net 3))
 (via (at 134.62 93.98) (size 2) (drill 0.8) (layers F.Cu B.Cu) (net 3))
 (segment (start 132.08 101.6) (end 132.08 101.6) (width 2) (layer B.Cu) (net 3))
 (segment (start 144.78 101.6) (end 132.08 101.6) (width 2) (layer B.Cu) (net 3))
 (segment (start 132.08 93.98) (end 124.46 93.98) (width 2) (layer B.Cu) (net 3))
 (via (at 132.08 93.98) (size 2) (drill 0.8) (layers F.Cu B.Cu) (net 3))
 (segment (start 132.08 101.6) (end 124.46 101.6) (width 2) (layer B.Cu) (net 3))
 (via (at 132.08 101.6) (size 2) (drill 0.8) (layers F.Cu B.Cu) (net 3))
 (segment (start 132.08 93.98) (end 132.08 101.6) (width 1) (layer F.Cu) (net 3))
 (segment (start 154.94 78.7) (end 172.72 78.74) (width 2) (layer B.Cu) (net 3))
 (segment (start 172.72 78.74) (end 182.88 78.74) (width 2) (layer B.Cu) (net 3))
 (segment (start 182.88 78.74) (end 182.88 104.14) (width 1) (layer F.Cu) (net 3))
 (segment (start 187.96 104.14) (end 182.88 104.14) (width 2) (layer B.Cu) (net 3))
 (segment (start 114.3 78.74) (end 109.22 78.74) (width 2) (layer B.Cu) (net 4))
 (via (at 177.8 91.44) (size 2) (drill 0.8) (layers F.Cu B.Cu) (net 1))
 (via (at 185.42 106.68) (size 2) (drill 0.8) (layers F.Cu B.Cu) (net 1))
 (via (at 134.62 111.76) (size 2) (drill 0.8) (layers F.Cu B.Cu) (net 1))
 (segment (start 152.4 91.44) (end 160.02 91.44) (width 2) (layer B.Cu) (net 1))
 (segment (start 144.78 109.22) (end 134.62 109.22) (width 2) (layer B.Cu) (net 1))
 (segment (start 134.62 109.22) (end 124.46 109.22) (width 2) (layer B.Cu) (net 1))
 (via (at 134.62 109.22) (size 2) (drill 0.8) (layers F.Cu B.Cu) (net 1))
 (segment (start 134.62 109.22) (end 134.62 111.76) (width 1) (layer F.Cu) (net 1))
 (segment (start 160.02 91.44) (end 172.72 91.44) (width 2) (layer B.Cu) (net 1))
 (segment (start 134.62 111.76) (end 177.8 111.76) (width 2) (layer B.Cu) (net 1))
 (segment (start 185.42 111.76) (end 185.42 111.76) (width 2) (layer B.Cu) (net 1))
 (via (at 185.42 111.76) (size 2) (drill 0.8) (layers F.Cu B.Cu) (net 1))
 (segment (start 187.96 106.68) (end 185.42 106.68) (width 2) (layer B.Cu) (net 1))
 (segment (start 185.42 106.68) (end 185.42 111.76) (width 1) (layer F.Cu) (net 1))
 (segment (start 177.8 111.76) (end 185.42 111.76) (width 2) (layer B.Cu) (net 1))
 (via (at 177.8 111.76) (size 2) (drill 0.8) (layers F.Cu B.Cu) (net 1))
 (segment (start 172.72 91.44) (end 177.8 91.44) (width 2) (layer B.Cu) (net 1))
 (segment (start 177.8 91.44) (end 177.8 111.76) (width 1) (layer F.Cu) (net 1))
 (segment (start 152.4 99.06) (end 162.56 99.06) (width 2) (layer B.Cu) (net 8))
 (segment (start 152.4 104.14) (end 162.56 104.14) (width 2) (layer B.Cu) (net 8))
 (segment (start 162.56 99.06) (end 172.72 99.06) (width 2) (layer B.Cu) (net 8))
 (via (at 162.56 99.06) (size 2) (drill 0.8) (layers F.Cu B.Cu) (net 8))
 (segment (start 162.56 104.14) (end 172.72 104.14) (width 2) (layer B.Cu) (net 8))
 (via (at 162.56 104.14) (size 2) (drill 0.8) (layers F.Cu B.Cu) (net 8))
 (segment (start 162.56 99.06) (end 162.56 104.14) (width 1) (layer F.Cu) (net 8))
 (segment (start 172.72 99.06) (end 187.96 99.06) (width 2) (layer B.Cu) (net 8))
 (via (at 180.34 106.68) (size 2) (drill 0.8) (layers F.Cu B.Cu) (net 7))
 (via (at 180.34 96.52) (size 2) (drill 0.8) (layers F.Cu B.Cu) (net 7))
 (via (at 162.56 114.3) (size 2) (drill 0.8) (layers F.Cu B.Cu) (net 7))
 (via (at 129.54 114.3) (size 2) (drill 0.8) (layers F.Cu B.Cu) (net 7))
 (segment (start 152.4 106.68) (end 162.56 106.68) (width 2) (layer B.Cu) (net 7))
 (segment (start 144.78 99.06) (end 129.54 99.06) (width 2) (layer B.Cu) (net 7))
 (segment (start 129.54 99.06) (end 124.46 99.06) (width 2) (layer B.Cu) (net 7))
 (segment (start 129.54 99.06) (end 129.54 99.06) (width 2) (layer B.Cu) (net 7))
 (via (at 129.54 99.06) (size 2) (drill 0.8) (layers F.Cu B.Cu) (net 7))
 (segment (start 129.54 99.06) (end 129.54 114.3) (width 1) (layer F.Cu) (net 7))
 (segment (start 162.56 106.68) (end 172.72 106.68) (width 2) (layer B.Cu) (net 7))
 (via (at 162.56 106.68) (size 2) (drill 0.8) (layers F.Cu B.Cu) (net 7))
 (segment (start 162.56 106.68) (end 162.56 114.3) (width 1) (layer F.Cu) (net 7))
 (segment (start 162.56 114.3) (end 129.54 114.3) (width 2) (layer B.Cu) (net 7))
 (segment (start 172.72 106.68) (end 180.34 106.68) (width 2) (layer B.Cu) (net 7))
 (segment (start 180.34 106.68) (end 180.34 96.52) (width 1) (layer F.Cu) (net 7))
 (segment (start 187.96 96.52) (end 180.34 96.52) (width 2) (layer B.Cu) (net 7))
 (via (at 119.38 116.84) (size 2) (drill 0.8) (layers F.Cu B.Cu) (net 9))
 (via (at 165.1 116.84) (size 2) (drill 0.8) (layers F.Cu B.Cu) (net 9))
 (segment (start 152.4 109.22) (end 165.1 109.22) (width 2) (layer B.Cu) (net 9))
 (segment (start 144.78 96.52) (end 124.46 96.52) (width 2) (layer B.Cu) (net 9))
 (segment (start 165.1 109.22) (end 172.72 109.22) (width 2) (layer B.Cu) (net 9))
 (via (at 165.1 109.22) (size 2) (drill 0.8) (layers F.Cu B.Cu) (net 9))
 (segment (start 119.38 96.52) (end 124.46 96.52) (width 2) (layer B.Cu) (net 9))
 (via (at 119.38 96.52) (size 2) (drill 0.8) (layers F.Cu B.Cu) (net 9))
 (segment (start 119.38 96.52) (end 119.38 116.84) (width 1) (layer F.Cu) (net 9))
 (segment (start 165.1 109.22) (end 165.1 116.84) (width 1) (layer F.Cu) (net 9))
 (segment (start 165.1 116.84) (end 119.38 116.84) (width 2) (layer B.Cu) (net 9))
 (segment (start 109.22 96.52) (end 119.38 96.52) (width 2) (layer B.Cu) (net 9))
 (segment (start 144.78 104.14) (end 124.46 104.14) (width 2) (layer B.Cu) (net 10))
 (segment (start 144.78 106.68) (end 124.46 106.68) (width 2) (layer B.Cu) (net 11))
 (segment (start 114.3 93.98) (end 109.22 93.98) (width 2) (layer B.Cu) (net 5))
 (segment (start 172.72 76.2) (end 167.64 76.2) (width 2) (layer B.Cu) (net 2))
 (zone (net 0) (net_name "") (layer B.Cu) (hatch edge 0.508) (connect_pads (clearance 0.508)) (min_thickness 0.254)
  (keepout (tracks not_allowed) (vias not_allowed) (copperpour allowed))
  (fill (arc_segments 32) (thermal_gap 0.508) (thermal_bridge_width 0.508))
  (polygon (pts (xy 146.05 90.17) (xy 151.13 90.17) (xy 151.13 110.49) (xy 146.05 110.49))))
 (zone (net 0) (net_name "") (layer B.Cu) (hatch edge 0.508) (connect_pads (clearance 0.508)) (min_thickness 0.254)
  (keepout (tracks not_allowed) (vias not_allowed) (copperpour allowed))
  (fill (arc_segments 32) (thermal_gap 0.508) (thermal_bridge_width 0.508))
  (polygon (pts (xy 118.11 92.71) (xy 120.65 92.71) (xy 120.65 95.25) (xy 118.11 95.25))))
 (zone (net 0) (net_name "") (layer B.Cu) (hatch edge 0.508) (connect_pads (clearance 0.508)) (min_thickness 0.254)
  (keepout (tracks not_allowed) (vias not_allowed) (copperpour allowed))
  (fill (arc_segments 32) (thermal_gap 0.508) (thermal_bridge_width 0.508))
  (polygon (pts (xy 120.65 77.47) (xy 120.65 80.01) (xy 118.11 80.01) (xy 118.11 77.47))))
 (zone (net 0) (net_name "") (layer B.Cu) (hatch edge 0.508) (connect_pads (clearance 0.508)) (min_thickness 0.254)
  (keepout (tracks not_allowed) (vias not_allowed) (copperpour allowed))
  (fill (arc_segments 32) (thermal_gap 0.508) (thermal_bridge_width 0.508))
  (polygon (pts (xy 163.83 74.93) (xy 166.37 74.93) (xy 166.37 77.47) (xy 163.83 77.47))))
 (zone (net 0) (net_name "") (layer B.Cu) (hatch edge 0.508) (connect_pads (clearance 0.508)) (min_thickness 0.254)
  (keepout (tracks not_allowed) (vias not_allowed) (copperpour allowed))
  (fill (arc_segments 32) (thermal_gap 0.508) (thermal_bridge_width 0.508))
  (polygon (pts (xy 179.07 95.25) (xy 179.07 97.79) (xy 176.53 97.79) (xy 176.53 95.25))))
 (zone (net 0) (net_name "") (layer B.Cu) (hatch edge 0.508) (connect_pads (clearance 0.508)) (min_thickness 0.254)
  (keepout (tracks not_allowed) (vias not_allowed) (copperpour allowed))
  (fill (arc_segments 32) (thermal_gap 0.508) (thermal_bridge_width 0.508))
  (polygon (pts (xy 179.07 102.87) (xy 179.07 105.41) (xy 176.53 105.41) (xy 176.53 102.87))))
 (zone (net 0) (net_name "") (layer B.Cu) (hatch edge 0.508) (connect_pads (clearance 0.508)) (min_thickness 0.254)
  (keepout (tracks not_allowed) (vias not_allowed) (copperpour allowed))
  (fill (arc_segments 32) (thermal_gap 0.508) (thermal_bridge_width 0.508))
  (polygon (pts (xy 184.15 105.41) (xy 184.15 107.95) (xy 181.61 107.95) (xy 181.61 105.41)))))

